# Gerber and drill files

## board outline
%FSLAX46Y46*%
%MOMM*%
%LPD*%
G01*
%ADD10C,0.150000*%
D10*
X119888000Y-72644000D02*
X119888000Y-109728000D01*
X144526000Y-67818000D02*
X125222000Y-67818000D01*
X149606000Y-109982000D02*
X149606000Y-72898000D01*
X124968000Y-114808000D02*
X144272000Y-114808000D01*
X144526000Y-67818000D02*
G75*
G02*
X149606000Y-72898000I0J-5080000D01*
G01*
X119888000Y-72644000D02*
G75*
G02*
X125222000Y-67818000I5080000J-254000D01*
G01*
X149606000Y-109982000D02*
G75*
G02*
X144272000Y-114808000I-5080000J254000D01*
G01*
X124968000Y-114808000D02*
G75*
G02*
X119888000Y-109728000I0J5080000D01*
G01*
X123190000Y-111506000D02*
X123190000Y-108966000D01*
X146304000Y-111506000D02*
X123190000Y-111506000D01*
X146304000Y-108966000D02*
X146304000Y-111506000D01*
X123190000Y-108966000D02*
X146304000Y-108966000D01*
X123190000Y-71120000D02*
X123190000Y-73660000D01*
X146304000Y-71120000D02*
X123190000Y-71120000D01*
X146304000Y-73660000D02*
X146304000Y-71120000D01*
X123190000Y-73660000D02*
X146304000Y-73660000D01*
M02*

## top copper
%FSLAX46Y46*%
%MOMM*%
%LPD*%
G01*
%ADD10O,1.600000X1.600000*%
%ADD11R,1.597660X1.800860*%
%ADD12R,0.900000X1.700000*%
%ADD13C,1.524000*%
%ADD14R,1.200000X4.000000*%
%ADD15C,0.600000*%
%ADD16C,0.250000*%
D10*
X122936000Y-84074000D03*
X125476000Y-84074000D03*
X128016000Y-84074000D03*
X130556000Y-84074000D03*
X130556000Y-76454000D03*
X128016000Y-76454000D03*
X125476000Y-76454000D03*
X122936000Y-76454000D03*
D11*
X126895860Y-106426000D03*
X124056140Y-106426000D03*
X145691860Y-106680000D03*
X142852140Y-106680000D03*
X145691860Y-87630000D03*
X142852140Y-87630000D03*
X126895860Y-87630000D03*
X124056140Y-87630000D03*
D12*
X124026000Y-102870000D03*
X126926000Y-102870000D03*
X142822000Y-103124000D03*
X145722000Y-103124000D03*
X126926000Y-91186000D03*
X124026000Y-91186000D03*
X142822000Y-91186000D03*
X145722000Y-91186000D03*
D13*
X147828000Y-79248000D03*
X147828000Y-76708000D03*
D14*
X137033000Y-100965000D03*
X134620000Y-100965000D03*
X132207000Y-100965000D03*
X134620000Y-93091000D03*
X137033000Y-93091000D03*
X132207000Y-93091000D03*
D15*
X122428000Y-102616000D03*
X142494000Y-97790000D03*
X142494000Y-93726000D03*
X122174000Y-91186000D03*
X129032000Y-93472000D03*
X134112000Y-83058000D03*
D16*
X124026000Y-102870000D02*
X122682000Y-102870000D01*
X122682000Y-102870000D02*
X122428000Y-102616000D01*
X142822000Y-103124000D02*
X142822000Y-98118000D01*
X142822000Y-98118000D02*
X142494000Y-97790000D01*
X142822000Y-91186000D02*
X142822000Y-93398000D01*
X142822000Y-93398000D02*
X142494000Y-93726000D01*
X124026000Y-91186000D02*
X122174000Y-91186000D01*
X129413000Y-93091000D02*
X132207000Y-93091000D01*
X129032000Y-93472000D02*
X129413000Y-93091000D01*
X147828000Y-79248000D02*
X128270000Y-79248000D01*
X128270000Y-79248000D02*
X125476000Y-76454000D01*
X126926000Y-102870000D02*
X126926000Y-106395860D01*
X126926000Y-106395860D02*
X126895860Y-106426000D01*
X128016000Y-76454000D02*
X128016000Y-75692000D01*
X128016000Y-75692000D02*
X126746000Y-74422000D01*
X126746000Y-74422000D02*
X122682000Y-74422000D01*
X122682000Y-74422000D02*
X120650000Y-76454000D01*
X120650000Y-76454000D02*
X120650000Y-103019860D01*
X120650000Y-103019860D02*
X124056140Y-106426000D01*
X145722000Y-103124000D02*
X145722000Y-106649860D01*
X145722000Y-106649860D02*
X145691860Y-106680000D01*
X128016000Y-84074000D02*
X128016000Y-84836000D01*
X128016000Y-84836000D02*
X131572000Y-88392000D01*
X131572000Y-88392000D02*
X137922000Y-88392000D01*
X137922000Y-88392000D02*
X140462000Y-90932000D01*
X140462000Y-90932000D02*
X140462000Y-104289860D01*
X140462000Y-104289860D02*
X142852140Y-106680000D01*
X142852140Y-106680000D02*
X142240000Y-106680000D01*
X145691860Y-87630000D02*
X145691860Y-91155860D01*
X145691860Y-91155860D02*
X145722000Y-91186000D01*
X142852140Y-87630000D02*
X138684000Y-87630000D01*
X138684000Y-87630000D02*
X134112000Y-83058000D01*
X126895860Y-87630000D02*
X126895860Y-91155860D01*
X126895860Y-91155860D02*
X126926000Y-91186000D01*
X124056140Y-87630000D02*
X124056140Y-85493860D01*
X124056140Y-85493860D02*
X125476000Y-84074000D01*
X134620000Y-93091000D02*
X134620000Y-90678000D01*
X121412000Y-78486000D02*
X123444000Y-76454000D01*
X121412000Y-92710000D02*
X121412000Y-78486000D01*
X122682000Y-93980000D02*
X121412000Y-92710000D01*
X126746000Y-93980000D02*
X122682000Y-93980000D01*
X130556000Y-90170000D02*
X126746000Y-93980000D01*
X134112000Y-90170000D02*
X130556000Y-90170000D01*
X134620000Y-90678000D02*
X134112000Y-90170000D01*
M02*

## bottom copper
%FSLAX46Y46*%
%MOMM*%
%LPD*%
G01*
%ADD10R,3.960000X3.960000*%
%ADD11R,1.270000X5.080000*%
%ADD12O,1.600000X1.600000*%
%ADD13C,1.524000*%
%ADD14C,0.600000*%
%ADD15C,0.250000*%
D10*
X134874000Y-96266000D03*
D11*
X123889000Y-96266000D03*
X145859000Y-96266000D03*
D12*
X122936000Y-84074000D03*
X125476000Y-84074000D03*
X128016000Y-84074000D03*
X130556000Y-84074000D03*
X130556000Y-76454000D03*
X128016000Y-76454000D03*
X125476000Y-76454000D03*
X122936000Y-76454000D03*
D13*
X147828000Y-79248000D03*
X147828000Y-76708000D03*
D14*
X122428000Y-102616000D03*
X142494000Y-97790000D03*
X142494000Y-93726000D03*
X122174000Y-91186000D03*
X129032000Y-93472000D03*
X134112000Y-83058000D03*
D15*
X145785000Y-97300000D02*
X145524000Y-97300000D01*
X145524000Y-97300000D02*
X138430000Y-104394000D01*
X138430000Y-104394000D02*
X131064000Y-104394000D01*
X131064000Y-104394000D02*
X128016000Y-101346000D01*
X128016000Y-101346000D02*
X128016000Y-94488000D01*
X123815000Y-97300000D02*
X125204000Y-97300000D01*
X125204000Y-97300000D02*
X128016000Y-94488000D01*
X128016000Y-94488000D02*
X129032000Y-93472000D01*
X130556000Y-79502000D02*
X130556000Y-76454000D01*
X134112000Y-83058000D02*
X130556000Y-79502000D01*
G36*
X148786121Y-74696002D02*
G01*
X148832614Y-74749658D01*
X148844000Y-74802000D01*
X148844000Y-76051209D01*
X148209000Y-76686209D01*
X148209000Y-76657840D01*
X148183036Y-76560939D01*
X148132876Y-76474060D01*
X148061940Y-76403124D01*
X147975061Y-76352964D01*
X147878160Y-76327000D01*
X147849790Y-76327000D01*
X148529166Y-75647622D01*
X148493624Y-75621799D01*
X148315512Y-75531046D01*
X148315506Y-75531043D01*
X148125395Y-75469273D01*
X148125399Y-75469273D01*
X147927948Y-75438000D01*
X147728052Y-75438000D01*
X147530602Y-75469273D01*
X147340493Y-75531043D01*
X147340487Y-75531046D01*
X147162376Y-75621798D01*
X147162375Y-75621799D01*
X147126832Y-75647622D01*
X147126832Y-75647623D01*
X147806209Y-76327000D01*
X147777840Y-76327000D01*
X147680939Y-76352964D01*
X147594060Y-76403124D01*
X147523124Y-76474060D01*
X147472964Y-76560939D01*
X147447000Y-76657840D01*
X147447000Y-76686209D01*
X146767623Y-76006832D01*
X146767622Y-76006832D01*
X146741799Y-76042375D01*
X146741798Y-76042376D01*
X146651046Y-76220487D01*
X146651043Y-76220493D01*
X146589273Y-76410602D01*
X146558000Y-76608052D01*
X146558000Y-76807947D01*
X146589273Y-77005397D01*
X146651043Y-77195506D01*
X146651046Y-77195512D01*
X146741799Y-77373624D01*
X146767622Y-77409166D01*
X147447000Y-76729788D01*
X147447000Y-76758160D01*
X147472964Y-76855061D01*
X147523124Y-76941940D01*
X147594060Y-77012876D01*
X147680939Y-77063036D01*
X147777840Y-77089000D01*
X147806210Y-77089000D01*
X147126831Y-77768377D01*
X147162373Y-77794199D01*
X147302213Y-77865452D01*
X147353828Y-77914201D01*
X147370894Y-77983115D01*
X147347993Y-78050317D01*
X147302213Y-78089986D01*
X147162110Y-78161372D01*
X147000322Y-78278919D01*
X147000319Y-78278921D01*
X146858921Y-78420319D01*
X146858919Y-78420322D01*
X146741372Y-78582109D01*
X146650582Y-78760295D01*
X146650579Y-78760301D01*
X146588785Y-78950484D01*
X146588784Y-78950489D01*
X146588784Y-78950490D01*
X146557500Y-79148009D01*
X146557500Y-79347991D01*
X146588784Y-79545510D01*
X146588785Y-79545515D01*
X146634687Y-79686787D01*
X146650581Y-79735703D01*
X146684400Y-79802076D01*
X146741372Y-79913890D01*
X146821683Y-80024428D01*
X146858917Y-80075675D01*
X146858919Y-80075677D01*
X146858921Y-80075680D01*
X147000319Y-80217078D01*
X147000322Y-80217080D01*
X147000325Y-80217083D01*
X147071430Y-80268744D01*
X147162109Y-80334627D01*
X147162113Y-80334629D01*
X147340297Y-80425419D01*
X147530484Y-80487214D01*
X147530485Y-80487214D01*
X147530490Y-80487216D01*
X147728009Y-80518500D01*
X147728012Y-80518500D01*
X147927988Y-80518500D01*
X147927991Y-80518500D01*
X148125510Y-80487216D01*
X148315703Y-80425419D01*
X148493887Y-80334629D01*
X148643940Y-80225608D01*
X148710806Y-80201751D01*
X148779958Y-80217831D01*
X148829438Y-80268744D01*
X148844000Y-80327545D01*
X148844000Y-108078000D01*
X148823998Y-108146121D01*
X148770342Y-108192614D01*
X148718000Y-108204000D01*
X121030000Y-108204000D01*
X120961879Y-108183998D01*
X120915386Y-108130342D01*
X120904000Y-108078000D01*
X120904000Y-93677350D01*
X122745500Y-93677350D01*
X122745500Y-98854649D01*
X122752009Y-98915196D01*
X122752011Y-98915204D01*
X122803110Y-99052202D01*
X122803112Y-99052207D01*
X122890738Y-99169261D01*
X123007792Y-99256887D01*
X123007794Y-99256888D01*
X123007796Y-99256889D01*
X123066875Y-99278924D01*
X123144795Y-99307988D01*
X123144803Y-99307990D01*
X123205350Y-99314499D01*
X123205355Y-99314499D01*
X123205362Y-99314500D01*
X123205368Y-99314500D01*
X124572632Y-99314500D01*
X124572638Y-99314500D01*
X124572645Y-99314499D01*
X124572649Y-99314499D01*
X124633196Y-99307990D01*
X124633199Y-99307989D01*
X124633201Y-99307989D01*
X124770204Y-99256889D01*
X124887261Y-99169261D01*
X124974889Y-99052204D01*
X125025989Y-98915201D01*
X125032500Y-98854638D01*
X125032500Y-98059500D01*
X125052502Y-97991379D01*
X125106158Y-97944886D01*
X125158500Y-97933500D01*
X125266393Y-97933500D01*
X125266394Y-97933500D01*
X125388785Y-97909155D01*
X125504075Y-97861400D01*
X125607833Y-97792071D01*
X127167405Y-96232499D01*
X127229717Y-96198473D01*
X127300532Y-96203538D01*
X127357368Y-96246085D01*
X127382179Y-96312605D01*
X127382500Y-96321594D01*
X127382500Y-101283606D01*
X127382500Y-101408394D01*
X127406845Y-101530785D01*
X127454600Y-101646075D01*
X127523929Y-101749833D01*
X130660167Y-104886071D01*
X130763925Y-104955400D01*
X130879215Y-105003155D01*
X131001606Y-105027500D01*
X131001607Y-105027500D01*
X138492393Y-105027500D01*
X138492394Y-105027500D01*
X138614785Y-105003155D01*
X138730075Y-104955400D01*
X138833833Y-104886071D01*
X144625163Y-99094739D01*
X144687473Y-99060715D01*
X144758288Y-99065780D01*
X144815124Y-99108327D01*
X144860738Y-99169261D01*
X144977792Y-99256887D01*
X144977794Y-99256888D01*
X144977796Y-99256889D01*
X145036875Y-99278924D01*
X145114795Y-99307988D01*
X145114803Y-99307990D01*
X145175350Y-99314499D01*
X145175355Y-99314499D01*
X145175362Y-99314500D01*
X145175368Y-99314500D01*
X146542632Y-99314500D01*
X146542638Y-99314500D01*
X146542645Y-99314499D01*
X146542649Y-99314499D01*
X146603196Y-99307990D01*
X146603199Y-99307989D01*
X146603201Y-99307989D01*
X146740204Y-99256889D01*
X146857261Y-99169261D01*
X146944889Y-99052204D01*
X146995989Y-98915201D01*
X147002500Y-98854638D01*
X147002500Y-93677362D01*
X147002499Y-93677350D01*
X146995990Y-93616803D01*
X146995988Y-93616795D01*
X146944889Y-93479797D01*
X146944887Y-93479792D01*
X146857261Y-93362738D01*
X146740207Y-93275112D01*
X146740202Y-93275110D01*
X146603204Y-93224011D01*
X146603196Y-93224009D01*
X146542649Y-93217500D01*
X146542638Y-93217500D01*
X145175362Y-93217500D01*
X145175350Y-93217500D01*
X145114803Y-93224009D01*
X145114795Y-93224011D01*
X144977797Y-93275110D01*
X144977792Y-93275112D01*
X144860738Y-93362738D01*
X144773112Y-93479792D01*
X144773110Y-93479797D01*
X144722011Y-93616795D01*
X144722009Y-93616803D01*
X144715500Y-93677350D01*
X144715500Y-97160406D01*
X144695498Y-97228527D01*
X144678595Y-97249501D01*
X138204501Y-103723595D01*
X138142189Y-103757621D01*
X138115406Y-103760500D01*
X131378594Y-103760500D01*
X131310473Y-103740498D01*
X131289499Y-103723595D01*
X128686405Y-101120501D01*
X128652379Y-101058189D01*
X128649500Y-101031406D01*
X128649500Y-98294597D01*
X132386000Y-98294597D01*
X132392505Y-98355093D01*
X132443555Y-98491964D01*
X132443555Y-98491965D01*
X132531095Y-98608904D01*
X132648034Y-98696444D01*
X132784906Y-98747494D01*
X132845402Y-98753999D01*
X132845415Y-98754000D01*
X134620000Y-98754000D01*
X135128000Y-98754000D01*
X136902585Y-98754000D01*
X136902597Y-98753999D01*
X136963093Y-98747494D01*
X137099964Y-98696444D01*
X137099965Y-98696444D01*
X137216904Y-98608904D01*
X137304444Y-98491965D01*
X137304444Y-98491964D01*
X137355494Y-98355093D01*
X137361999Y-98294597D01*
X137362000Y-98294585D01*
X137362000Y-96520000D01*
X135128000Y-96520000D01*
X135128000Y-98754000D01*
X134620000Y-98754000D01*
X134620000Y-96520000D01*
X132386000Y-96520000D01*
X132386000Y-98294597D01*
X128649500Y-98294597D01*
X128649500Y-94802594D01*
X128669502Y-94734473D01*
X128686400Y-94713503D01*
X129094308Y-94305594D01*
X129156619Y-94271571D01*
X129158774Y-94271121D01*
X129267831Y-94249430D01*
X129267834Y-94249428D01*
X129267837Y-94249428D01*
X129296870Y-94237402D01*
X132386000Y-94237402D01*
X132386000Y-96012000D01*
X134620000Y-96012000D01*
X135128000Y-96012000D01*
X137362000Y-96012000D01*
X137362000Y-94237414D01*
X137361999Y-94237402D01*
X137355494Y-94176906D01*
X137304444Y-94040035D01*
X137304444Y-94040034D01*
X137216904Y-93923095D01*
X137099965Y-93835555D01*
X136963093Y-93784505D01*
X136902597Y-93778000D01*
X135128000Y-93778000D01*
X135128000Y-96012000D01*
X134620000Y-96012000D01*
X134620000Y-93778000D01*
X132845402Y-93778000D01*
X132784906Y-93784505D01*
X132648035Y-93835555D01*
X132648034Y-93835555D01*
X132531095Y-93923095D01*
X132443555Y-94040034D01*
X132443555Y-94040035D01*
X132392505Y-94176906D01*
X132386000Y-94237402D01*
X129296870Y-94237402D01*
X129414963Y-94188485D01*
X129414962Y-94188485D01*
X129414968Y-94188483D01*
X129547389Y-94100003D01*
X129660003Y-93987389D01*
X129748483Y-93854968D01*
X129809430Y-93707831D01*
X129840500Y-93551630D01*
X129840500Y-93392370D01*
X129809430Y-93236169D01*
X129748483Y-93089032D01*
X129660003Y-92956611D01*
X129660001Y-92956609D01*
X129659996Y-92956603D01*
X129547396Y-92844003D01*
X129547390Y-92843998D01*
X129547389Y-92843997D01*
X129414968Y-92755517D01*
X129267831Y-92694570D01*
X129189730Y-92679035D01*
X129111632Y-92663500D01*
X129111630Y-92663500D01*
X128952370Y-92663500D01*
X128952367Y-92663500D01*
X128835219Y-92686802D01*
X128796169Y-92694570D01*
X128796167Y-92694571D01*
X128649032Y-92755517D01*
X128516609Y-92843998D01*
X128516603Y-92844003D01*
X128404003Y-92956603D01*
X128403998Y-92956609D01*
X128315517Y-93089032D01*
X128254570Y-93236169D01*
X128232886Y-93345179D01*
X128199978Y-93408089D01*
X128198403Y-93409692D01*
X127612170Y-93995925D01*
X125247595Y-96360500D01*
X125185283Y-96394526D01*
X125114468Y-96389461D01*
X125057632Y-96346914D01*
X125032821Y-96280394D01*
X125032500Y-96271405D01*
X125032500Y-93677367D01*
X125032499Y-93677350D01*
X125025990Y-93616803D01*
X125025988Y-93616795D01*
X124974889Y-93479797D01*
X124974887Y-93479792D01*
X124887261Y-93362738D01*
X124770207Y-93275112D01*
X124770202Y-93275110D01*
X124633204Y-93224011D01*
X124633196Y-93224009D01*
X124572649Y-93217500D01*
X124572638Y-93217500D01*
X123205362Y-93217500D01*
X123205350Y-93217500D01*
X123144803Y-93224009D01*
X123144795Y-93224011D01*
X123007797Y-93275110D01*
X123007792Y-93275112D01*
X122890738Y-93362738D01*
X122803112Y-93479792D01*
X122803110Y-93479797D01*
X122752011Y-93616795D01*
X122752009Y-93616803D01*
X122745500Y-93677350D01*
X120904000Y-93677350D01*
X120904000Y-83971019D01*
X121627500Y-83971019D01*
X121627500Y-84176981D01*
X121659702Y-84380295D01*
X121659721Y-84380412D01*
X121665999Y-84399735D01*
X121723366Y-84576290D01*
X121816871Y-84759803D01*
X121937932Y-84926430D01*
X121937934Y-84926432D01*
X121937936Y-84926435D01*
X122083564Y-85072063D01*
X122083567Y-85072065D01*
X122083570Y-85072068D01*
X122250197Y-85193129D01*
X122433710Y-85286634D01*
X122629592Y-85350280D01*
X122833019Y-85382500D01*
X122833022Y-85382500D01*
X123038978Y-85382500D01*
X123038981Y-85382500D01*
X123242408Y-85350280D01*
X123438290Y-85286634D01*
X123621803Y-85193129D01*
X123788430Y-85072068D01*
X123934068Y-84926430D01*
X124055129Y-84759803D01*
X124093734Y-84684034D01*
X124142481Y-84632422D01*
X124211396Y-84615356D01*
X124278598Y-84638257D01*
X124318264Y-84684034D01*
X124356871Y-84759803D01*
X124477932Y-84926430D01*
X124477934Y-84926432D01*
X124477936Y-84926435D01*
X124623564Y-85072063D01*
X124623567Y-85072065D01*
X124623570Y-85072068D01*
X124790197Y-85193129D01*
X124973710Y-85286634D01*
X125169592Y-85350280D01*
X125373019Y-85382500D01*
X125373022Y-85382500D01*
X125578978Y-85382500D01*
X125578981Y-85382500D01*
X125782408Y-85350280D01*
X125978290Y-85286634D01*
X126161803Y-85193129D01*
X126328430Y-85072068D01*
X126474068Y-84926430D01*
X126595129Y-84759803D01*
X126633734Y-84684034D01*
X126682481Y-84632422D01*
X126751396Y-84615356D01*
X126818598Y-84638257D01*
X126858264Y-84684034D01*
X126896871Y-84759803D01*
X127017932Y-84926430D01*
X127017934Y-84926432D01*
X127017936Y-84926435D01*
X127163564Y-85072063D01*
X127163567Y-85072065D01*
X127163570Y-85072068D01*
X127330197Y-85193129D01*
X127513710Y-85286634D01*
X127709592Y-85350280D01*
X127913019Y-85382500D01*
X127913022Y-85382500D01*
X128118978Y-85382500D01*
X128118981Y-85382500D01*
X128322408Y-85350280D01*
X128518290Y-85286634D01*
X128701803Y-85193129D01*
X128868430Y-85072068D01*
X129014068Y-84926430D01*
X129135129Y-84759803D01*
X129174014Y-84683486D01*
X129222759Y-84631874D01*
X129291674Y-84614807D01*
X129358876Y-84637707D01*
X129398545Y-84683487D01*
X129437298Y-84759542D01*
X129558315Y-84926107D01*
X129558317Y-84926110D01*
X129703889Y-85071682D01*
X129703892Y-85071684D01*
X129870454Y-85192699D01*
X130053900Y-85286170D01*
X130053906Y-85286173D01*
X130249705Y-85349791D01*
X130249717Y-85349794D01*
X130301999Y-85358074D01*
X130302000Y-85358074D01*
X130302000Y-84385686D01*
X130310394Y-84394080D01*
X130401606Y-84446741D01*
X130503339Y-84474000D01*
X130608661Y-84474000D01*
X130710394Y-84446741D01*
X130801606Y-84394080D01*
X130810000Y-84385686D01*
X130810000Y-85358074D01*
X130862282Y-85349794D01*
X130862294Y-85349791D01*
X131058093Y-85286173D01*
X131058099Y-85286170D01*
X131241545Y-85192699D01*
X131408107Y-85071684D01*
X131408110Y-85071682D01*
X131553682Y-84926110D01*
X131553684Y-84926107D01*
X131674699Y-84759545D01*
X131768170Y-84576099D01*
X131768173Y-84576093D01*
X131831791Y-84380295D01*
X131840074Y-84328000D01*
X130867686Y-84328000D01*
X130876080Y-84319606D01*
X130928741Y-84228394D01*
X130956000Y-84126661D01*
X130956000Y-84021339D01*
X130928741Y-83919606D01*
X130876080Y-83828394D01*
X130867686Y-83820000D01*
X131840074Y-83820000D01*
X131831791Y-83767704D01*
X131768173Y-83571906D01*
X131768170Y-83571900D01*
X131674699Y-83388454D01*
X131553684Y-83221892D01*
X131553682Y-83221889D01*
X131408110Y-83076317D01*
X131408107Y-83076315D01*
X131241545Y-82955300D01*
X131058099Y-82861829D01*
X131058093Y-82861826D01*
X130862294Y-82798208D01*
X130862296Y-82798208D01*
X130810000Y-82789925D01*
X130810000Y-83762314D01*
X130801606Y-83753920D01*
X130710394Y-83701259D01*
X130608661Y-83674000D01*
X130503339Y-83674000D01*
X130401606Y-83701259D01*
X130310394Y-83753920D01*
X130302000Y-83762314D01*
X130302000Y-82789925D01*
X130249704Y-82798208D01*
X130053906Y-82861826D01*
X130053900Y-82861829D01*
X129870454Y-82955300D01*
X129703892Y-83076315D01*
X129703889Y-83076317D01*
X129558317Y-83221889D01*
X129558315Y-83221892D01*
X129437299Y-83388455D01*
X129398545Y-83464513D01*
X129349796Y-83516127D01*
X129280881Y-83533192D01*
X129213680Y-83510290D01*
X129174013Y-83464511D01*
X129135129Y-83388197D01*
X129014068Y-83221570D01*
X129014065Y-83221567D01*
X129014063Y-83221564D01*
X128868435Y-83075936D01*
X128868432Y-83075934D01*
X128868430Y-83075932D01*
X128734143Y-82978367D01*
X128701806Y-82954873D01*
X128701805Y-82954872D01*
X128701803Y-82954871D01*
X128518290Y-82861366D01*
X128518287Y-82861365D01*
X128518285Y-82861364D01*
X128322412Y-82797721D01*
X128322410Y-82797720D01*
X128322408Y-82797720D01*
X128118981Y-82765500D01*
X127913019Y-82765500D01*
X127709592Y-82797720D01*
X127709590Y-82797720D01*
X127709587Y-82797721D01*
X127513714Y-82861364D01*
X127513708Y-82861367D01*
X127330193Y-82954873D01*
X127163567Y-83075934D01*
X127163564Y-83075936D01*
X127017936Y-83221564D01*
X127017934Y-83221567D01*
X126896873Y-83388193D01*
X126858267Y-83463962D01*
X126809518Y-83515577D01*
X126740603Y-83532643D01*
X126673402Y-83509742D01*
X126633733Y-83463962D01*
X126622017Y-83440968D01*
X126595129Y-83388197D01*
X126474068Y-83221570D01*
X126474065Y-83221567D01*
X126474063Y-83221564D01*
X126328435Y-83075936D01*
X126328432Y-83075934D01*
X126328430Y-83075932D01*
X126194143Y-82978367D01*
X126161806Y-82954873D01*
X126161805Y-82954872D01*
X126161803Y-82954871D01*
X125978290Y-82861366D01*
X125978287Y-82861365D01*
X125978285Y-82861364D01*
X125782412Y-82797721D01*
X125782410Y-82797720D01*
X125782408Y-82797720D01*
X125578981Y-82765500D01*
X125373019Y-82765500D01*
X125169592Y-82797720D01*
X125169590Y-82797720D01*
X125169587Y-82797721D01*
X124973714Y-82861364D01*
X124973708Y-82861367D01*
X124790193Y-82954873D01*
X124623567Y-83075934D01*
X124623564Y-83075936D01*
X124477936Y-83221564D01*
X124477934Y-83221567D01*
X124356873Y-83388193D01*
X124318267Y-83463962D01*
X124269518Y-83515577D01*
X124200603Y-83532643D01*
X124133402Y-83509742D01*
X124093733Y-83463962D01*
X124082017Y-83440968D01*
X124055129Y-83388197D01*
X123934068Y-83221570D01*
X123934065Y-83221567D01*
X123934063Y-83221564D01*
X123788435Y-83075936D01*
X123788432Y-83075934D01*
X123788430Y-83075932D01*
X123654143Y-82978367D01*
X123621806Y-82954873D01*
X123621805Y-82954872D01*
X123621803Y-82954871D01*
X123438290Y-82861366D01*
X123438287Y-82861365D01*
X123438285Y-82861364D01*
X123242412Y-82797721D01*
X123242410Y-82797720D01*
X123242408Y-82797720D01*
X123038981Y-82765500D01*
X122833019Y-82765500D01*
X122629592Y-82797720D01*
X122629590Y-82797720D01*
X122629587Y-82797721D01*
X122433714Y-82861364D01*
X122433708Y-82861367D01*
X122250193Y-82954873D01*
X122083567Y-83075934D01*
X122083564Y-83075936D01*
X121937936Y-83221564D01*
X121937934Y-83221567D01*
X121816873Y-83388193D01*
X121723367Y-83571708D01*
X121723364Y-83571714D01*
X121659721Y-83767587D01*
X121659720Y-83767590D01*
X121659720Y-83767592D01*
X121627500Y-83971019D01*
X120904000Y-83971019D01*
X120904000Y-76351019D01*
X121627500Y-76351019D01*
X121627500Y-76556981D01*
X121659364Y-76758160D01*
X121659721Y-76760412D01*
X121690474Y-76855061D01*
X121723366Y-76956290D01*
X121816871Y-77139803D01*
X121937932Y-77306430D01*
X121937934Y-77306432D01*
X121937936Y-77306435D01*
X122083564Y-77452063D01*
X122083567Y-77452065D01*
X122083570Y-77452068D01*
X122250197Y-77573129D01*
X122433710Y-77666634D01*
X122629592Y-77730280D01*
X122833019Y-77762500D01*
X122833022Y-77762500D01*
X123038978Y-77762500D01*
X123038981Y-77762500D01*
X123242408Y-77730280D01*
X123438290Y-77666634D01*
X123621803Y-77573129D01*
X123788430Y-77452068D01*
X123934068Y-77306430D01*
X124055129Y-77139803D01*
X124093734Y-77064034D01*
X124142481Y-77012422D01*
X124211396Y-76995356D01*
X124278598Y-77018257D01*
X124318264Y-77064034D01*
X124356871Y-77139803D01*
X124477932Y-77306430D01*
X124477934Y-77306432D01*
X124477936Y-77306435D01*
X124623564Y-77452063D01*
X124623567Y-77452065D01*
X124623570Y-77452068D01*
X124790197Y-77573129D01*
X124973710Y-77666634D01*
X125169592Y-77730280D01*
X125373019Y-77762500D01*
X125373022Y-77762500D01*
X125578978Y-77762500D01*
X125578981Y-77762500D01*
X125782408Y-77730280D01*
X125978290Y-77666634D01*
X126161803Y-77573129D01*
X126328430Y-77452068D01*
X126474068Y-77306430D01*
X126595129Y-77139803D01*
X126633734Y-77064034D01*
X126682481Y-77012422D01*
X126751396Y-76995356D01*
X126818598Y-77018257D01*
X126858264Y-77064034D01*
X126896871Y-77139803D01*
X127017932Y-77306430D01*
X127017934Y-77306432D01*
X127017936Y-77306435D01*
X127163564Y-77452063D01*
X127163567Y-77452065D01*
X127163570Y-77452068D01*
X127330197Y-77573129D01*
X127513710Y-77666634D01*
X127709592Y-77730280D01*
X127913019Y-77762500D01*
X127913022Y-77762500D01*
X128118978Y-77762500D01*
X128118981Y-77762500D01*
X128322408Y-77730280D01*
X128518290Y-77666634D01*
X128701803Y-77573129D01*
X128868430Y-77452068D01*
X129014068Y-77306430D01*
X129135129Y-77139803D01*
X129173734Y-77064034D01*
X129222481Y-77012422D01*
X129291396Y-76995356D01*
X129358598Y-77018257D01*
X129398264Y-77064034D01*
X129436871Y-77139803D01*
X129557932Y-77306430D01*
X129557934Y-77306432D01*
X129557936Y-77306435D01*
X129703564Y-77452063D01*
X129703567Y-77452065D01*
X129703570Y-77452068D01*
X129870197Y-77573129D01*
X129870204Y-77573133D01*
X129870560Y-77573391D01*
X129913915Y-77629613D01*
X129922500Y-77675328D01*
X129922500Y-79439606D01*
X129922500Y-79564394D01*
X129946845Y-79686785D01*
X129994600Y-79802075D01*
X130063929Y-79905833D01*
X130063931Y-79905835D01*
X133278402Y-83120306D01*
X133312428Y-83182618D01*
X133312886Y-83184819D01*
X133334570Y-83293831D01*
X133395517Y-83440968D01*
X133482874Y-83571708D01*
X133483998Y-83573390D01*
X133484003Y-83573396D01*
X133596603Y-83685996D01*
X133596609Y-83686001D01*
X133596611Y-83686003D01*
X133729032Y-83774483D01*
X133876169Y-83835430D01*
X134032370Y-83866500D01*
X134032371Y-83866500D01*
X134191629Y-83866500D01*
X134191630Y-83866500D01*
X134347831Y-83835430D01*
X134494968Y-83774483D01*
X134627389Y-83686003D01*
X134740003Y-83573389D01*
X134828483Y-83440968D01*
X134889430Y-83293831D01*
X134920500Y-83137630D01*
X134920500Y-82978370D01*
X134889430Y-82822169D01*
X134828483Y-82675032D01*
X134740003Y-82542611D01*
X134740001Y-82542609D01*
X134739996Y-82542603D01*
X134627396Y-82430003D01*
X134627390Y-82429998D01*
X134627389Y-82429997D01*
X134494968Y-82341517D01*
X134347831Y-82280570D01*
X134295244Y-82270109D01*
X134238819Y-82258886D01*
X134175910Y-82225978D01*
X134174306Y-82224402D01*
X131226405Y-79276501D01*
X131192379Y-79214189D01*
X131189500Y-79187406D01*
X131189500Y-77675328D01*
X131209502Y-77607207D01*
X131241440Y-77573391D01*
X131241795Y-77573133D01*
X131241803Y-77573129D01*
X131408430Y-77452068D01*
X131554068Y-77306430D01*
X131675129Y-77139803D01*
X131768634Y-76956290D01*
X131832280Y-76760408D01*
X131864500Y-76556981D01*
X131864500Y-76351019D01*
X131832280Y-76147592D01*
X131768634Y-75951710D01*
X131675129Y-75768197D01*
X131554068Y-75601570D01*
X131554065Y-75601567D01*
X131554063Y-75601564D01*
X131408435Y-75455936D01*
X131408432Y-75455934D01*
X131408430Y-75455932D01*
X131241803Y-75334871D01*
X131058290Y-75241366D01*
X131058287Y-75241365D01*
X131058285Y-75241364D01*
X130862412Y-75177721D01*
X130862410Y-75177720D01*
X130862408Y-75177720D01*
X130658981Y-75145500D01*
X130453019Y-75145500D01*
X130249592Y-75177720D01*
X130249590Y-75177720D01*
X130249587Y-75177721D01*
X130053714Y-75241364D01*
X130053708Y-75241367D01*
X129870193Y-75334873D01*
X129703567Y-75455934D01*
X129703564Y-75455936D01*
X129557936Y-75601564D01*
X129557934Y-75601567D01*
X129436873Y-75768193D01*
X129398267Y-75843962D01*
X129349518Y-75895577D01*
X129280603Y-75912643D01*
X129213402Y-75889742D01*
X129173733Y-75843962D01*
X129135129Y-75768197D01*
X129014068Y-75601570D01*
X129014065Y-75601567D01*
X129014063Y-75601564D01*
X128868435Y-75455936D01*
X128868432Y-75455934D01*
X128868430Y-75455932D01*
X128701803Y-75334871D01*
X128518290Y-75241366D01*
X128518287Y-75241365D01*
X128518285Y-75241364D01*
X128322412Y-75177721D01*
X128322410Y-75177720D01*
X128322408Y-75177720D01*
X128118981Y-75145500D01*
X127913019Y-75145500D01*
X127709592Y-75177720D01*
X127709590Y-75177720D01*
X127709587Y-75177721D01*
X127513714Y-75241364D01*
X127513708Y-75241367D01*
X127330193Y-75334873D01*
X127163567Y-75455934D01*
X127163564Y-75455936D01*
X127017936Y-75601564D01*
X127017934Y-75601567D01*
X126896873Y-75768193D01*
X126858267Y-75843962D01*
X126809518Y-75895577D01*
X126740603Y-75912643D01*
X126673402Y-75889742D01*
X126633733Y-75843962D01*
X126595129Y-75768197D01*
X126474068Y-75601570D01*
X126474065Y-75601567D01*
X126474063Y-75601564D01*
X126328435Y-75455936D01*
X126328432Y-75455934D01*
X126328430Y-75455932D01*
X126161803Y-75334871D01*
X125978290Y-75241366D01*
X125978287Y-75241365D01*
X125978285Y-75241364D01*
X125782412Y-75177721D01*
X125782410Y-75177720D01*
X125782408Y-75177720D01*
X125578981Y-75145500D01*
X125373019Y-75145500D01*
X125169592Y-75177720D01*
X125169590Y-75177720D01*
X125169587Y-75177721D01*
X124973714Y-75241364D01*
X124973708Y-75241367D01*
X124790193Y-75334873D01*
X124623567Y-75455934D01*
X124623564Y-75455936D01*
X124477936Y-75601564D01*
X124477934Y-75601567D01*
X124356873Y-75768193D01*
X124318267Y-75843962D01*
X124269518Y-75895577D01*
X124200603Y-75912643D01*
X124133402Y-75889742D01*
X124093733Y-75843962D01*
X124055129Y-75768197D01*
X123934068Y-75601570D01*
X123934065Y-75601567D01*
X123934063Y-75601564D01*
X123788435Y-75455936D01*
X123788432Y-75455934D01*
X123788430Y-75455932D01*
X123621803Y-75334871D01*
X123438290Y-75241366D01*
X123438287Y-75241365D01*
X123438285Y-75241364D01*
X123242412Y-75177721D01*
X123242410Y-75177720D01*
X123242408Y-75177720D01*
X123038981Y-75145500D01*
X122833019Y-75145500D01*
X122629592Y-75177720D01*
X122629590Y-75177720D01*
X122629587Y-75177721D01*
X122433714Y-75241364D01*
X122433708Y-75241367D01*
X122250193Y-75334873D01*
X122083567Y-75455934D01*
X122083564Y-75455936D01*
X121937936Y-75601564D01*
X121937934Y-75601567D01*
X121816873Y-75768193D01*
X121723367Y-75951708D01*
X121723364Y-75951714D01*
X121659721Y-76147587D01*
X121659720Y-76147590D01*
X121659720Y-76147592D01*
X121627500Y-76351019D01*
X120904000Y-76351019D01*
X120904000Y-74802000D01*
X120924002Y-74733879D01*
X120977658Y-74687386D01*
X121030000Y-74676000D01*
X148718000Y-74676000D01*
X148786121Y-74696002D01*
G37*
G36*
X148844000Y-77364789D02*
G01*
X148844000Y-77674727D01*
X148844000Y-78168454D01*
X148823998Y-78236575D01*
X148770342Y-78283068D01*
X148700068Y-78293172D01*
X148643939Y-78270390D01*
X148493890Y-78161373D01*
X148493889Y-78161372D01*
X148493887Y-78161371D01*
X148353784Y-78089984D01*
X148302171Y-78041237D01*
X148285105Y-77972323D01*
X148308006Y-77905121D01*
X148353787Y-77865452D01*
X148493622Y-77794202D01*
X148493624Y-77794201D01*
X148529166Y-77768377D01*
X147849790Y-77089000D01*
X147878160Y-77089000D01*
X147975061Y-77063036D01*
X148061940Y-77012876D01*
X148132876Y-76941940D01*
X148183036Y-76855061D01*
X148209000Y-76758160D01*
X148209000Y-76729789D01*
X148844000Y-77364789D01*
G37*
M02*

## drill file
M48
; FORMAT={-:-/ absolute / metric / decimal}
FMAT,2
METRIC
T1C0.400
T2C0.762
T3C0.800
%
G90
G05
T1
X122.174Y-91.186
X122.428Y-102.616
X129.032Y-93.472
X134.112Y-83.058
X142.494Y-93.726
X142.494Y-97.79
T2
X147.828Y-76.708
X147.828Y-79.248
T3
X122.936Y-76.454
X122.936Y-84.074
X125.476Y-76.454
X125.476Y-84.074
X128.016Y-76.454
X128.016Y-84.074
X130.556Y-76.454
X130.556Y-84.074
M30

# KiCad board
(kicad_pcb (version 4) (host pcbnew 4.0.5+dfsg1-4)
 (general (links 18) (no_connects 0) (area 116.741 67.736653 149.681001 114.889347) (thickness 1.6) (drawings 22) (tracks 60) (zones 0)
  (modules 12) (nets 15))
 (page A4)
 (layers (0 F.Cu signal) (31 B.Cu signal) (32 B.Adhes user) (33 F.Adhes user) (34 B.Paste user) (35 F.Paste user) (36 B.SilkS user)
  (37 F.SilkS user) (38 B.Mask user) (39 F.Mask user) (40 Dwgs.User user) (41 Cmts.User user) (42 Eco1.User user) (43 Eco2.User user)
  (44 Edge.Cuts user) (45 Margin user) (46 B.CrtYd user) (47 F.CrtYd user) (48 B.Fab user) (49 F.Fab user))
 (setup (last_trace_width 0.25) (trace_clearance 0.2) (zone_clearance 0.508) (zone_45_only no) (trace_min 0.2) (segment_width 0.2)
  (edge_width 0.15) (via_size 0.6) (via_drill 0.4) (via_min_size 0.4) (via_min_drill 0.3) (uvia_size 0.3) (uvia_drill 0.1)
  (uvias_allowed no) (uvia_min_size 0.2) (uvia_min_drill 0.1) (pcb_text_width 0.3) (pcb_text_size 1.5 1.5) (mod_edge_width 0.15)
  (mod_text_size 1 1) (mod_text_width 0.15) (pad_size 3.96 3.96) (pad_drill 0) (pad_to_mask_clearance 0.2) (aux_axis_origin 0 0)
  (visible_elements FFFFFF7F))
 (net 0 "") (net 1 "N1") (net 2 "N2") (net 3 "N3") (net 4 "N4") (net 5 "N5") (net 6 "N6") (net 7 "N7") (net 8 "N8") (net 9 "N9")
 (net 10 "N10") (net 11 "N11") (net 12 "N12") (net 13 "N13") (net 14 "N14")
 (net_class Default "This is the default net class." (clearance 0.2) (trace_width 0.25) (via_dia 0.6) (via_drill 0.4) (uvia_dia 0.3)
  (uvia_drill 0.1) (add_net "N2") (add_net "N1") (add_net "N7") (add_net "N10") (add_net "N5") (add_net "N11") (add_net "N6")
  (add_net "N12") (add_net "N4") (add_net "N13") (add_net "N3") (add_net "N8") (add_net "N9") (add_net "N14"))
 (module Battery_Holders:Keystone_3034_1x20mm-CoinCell (layer B.Cu) (at 134.874 96.266 180)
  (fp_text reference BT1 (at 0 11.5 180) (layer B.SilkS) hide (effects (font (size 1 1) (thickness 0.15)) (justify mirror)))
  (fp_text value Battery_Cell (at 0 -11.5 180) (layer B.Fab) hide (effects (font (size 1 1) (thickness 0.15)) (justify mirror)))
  (pad 2 smd rect (at 0 0 180) (size 3.96 3.96) (layers B.Cu B.Paste B.Mask) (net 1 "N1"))
  (pad 1 smd rect (at 10.985 0 180) (size 1.27 5.08) (layers B.Cu B.Paste B.Mask) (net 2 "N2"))
  (pad 1 smd rect (at -10.985 0 180) (size 1.27 5.08) (layers B.Cu B.Paste B.Mask) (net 2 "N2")))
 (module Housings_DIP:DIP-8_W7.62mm (layer F.Cu) (at 122.936 84.074 90)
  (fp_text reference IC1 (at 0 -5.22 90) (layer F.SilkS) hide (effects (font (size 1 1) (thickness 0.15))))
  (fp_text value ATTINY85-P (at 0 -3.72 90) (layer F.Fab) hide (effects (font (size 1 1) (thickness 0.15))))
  (pad 1 thru_hole oval (at 0 0 90) (size 1.6 1.6) (drill 0.8) (layers *.Cu *.Mask) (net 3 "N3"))
  (pad 2 thru_hole oval (at 0 2.54 90) (size 1.6 1.6) (drill 0.8) (layers *.Cu *.Mask) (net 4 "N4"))
  (pad 3 thru_hole oval (at 0 5.08 90) (size 1.6 1.6) (drill 0.8) (layers *.Cu *.Mask) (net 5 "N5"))
  (pad 4 thru_hole oval (at 0 7.62 90) (size 1.6 1.6) (drill 0.8) (layers *.Cu *.Mask) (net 1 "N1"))
  (pad 5 thru_hole oval (at 7.62 7.62 90) (size 1.6 1.6) (drill 0.8) (layers *.Cu *.Mask) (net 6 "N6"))
  (pad 6 thru_hole oval (at 7.62 5.08 90) (size 1.6 1.6) (drill 0.8) (layers *.Cu *.Mask) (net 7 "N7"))
  (pad 7 thru_hole oval (at 7.62 2.54 90) (size 1.6 1.6) (drill 0.8) (layers *.Cu *.Mask) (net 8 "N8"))
  (pad 8 thru_hole oval (at 7.62 0 90) (size 1.6 1.6) (drill 0.8) (layers *.Cu *.Mask) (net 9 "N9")))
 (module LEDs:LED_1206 (layer F.Cu) (at 125.476 106.426)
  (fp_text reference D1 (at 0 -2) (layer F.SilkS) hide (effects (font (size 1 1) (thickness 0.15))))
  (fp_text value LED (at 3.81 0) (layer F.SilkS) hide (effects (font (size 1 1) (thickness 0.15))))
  (pad 2 smd rect (at 1.41986 0 180) (size 1.59766 1.80086) (layers F.Cu F.Paste F.Mask) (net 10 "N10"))
  (pad 1 smd rect (at -1.41986 0 180) (size 1.59766 1.80086) (layers F.Cu F.Paste F.Mask) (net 7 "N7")))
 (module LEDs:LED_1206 (layer F.Cu) (at 144.272 106.68)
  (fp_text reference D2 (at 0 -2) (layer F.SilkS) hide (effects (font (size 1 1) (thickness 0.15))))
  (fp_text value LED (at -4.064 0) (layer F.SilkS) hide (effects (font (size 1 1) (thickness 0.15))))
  (pad 2 smd rect (at 1.41986 0 180) (size 1.59766 1.80086) (layers F.Cu F.Paste F.Mask) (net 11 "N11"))
  (pad 1 smd rect (at -1.41986 0 180) (size 1.59766 1.80086) (layers F.Cu F.Paste F.Mask) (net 5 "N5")))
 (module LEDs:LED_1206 (layer F.Cu) (at 144.272 87.63)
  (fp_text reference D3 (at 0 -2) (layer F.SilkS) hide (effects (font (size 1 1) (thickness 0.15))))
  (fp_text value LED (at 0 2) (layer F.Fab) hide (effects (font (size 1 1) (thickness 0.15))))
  (pad 2 smd rect (at 1.41986 0 180) (size 1.59766 1.80086) (layers F.Cu F.Paste F.Mask) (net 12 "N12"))
  (pad 1 smd rect (at -1.41986 0 180) (size 1.59766 1.80086) (layers F.Cu F.Paste F.Mask) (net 6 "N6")))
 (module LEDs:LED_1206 (layer F.Cu) (at 125.476 87.63)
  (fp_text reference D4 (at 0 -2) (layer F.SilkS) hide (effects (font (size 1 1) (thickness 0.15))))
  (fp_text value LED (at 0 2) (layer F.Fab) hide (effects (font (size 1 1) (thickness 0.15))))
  (pad 2 smd rect (at 1.41986 0 180) (size 1.59766 1.80086) (layers F.Cu F.Paste F.Mask) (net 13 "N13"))
  (pad 1 smd rect (at -1.41986 0 180) (size 1.59766 1.80086) (layers F.Cu F.Paste F.Mask) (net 4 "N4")))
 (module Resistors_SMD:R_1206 (layer F.Cu) (at 125.476 102.87)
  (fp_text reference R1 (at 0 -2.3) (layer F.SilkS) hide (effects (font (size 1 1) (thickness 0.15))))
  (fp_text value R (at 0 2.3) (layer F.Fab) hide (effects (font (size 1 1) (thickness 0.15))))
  (pad 1 smd rect (at -1.45 0) (size 0.9 1.7) (layers F.Cu F.Paste F.Mask) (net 1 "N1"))
  (pad 2 smd rect (at 1.45 0) (size 0.9 1.7) (layers F.Cu F.Paste F.Mask) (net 10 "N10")))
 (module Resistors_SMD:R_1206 (layer F.Cu) (at 144.272 103.124)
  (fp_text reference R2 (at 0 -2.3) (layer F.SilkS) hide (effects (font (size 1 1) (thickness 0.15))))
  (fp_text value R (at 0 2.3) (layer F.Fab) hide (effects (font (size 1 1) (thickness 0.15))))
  (pad 1 smd rect (at -1.45 0) (size 0.9 1.7) (layers F.Cu F.Paste F.Mask) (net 1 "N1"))
  (pad 2 smd rect (at 1.45 0) (size 0.9 1.7) (layers F.Cu F.Paste F.Mask) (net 11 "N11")))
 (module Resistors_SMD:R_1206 (layer F.Cu) (at 125.476 91.186 180)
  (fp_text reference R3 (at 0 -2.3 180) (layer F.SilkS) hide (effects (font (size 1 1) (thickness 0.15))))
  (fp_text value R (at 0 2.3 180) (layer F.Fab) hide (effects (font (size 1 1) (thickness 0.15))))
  (pad 1 smd rect (at -1.45 0 180) (size 0.9 1.7) (layers F.Cu F.Paste F.Mask) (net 13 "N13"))
  (pad 2 smd rect (at 1.45 0 180) (size 0.9 1.7) (layers F.Cu F.Paste F.Mask) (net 1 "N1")))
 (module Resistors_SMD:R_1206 (layer F.Cu) (at 144.272 91.186)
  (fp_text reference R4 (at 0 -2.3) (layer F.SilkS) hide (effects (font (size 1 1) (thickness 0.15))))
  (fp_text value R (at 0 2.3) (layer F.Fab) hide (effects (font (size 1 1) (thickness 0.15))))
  (pad 1 smd rect (at -1.45 0) (size 0.9 1.7) (layers F.Cu F.Paste F.Mask) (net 1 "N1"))
  (pad 2 smd rect (at 1.45 0) (size 0.9 1.7) (layers F.Cu F.Paste F.Mask) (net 12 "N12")))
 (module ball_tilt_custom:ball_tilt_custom (layer F.Cu) (at 147.828 77.978 180)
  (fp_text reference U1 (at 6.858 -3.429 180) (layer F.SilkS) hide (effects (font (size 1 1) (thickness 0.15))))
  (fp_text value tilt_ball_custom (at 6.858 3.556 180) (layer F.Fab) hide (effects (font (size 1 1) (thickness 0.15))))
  (pad 1 thru_hole circle (at 0 -1.27 180) (size 1.524 1.524) (drill 0.762) (layers *.Cu *.Mask) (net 8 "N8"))
  (pad 2 thru_hole circle (at 0 1.27 180) (size 1.524 1.524) (drill 0.762) (layers *.Cu *.Mask) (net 1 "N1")))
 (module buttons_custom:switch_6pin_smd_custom (layer F.Cu) (at 134.62 97.028)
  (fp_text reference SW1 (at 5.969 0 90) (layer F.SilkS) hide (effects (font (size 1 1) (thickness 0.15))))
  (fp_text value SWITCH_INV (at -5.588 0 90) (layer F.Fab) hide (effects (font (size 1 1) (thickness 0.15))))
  (pad 6 smd rect (at 2.413 3.937) (size 1.2 4) (layers F.Cu F.Paste F.Mask))
  (pad 5 smd rect (at 0 3.937) (size 1.2 4) (layers F.Cu F.Paste F.Mask))
  (pad 4 smd rect (at -2.413 3.937) (size 1.2 4) (layers F.Cu F.Paste F.Mask))
  (pad 2 smd rect (at 0 -3.937) (size 1.2 4) (layers F.Cu F.Paste F.Mask) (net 9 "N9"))
  (pad 3 smd rect (at 2.413 -3.937) (size 1.2 4) (layers F.Cu F.Paste F.Mask) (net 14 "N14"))
  (pad 1 smd rect (at -2.413 -3.937) (size 1.2 4) (layers F.Cu F.Paste F.Mask) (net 2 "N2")))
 (gr_line (start 119.888 72.644) (end 119.888 109.728) (angle 90) (layer Edge.Cuts) (width 0.15))
 (gr_line (start 144.526 67.818) (end 125.222 67.818) (angle 90) (layer Edge.Cuts) (width 0.15))
 (gr_line (start 149.606 109.982) (end 149.606 72.898) (angle 90) (layer Edge.Cuts) (width 0.15))
 (gr_line (start 124.968 114.808) (end 144.272 114.808) (angle 90) (layer Edge.Cuts) (width 0.15))
 (gr_arc (start 144.526 72.898) (end 144.526 67.818) (angle 90) (layer Edge.Cuts) (width 0.15))
 (gr_arc (start 124.968 72.898) (end 119.888 72.644) (angle 90) (layer Edge.Cuts) (width 0.15))
 (gr_arc (start 144.526 109.728) (end 149.606 109.982) (angle 90) (layer Edge.Cuts) (width 0.15))
 (gr_arc (start 124.968 109.728) (end 124.968 114.808) (angle 90) (layer Edge.Cuts) (width 0.15))
 (gr_line (start 123.19 111.506) (end 123.19 108.966) (angle 90) (layer Edge.Cuts) (width 0.15))
 (gr_line (start 146.304 111.506) (end 123.19 111.506) (angle 90) (layer Edge.Cuts) (width 0.15))
 (gr_line (start 146.304 108.966) (end 146.304 111.506) (angle 90) (layer Edge.Cuts) (width 0.15))
 (gr_line (start 123.19 108.966) (end 146.304 108.966) (angle 90) (layer Edge.Cuts) (width 0.15))
 (gr_line (start 123.19 71.12) (end 123.19 73.66) (angle 90) (layer Edge.Cuts) (width 0.15))
 (gr_line (start 146.304 71.12) (end 123.19 71.12) (angle 90) (layer Edge.Cuts) (width 0.15))
 (gr_line (start 146.304 73.66) (end 146.304 71.12) (angle 90) (layer Edge.Cuts) (width 0.15))
 (gr_line (start 123.19 73.66) (end 146.304 73.66) (angle 90) (layer Edge.Cuts) (width 0.15))
 (segment (start 124.026 102.87) (end 122.682 102.87) (width 0.25) (layer F.Cu) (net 1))
 (via (at 122.428 102.616) (size 0.6) (drill 0.4) (layers F.Cu B.Cu) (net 1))
 (segment (start 122.682 102.87) (end 122.428 102.616) (width 0.25) (layer F.Cu) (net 1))
 (segment (start 142.822 103.124) (end 142.822 98.118) (width 0.25) (layer F.Cu) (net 1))
 (via (at 142.494 97.79) (size 0.6) (drill 0.4) (layers F.Cu B.Cu) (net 1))
 (segment (start 142.822 98.118) (end 142.494 97.79) (width 0.25) (layer F.Cu) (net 1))
 (segment (start 142.822 91.186) (end 142.822 93.398) (width 0.25) (layer F.Cu) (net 1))
 (via (at 142.494 93.726) (size 0.6) (drill 0.4) (layers F.Cu B.Cu) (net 1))
 (segment (start 142.822 93.398) (end 142.494 93.726) (width 0.25) (layer F.Cu) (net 1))
 (segment (start 124.026 91.186) (end 122.174 91.186) (width 0.25) (layer F.Cu) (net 1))
 (via (at 122.174 91.186) (size 0.6) (drill 0.4) (layers F.Cu B.Cu) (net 1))
 (segment (start 145.785 97.3) (end 145.524 97.3) (width 0.25) (layer B.Cu) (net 2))
 (segment (start 145.524 97.3) (end 138.43 104.394) (width 0.25) (layer B.Cu) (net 2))
 (segment (start 138.43 104.394) (end 131.064 104.394) (width 0.25) (layer B.Cu) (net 2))
 (segment (start 131.064 104.394) (end 128.016 101.346) (width 0.25) (layer B.Cu) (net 2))
 (segment (start 128.016 101.346) (end 128.016 94.488) (width 0.25) (layer B.Cu) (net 2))
 (segment (start 123.815 97.3) (end 125.204 97.3) (width 0.25) (layer B.Cu) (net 2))
 (segment (start 129.413 93.091) (end 132.207 93.091) (width 0.25) (layer F.Cu) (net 2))
 (segment (start 129.032 93.472) (end 129.413 93.091) (width 0.25) (layer F.Cu) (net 2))
 (via (at 129.032 93.472) (size 0.6) (drill 0.4) (layers F.Cu B.Cu) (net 2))
 (segment (start 125.204 97.3) (end 128.016 94.488) (width 0.25) (layer B.Cu) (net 2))
 (segment (start 128.016 94.488) (end 129.032 93.472) (width 0.25) (layer B.Cu) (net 2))
 (segment (start 147.828 79.248) (end 128.27 79.248) (width 0.25) (layer F.Cu) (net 8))
 (segment (start 128.27 79.248) (end 125.476 76.454) (width 0.25) (layer F.Cu) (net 8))
 (segment (start 126.926 102.87) (end 126.926 106.39586) (width 0.25) (layer F.Cu) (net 10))
 (segment (start 126.926 106.39586) (end 126.89586 106.426) (width 0.25) (layer F.Cu) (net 10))
 (segment (start 128.016 76.454) (end 128.016 75.692) (width 0.25) (layer F.Cu) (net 7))
 (segment (start 128.016 75.692) (end 126.746 74.422) (width 0.25) (layer F.Cu) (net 7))
 (segment (start 126.746 74.422) (end 122.682 74.422) (width 0.25) (layer F.Cu) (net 7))
 (segment (start 122.682 74.422) (end 120.65 76.454) (width 0.25) (layer F.Cu) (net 7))
 (segment (start 120.65 76.454) (end 120.65 103.01986) (width 0.25) (layer F.Cu) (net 7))
 (segment (start 120.65 103.01986) (end 124.05614 106.426) (width 0.25) (layer F.Cu) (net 7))
 (segment (start 145.722 103.124) (end 145.722 106.64986) (width 0.25) (layer F.Cu) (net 11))
 (segment (start 145.722 106.64986) (end 145.69186 106.68) (width 0.25) (layer F.Cu) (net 11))
 (segment (start 128.016 84.074) (end 128.016 84.836) (width 0.25) (layer F.Cu) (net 5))
 (segment (start 128.016 84.836) (end 131.572 88.392) (width 0.25) (layer F.Cu) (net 5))
 (segment (start 131.572 88.392) (end 137.922 88.392) (width 0.25) (layer F.Cu) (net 5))
 (segment (start 137.922 88.392) (end 140.462 90.932) (width 0.25) (layer F.Cu) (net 5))
 (segment (start 140.462 90.932) (end 140.462 104.28986) (width 0.25) (layer F.Cu) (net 5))
 (segment (start 140.462 104.28986) (end 142.85214 106.68) (width 0.25) (layer F.Cu) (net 5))
 (segment (start 142.85214 106.68) (end 142.24 106.68) (width 0.25) (layer F.Cu) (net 5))
 (segment (start 145.69186 87.63) (end 145.69186 91.15586) (width 0.25) (layer F.Cu) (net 12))
 (segment (start 145.69186 91.15586) (end 145.722 91.186) (width 0.25) (layer F.Cu) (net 12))
 (segment (start 142.85214 87.63) (end 138.684 87.63) (width 0.25) (layer F.Cu) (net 6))
 (segment (start 130.556 79.502) (end 130.556 76.454) (width 0.25) (layer B.Cu) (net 6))
 (segment (start 134.112 83.058) (end 130.556 79.502) (width 0.25) (layer B.Cu) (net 6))
 (via (at 134.112 83.058) (size 0.6) (drill 0.4) (layers F.Cu B.Cu) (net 6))
 (segment (start 138.684 87.63) (end 134.112 83.058) (width 0.25) (layer F.Cu) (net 6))
 (segment (start 126.89586 87.63) (end 126.89586 91.15586) (width 0.25) (layer F.Cu) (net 13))
 (segment (start 126.89586 91.15586) (end 126.926 91.186) (width 0.25) (layer F.Cu) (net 13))
 (segment (start 124.05614 87.63) (end 124.05614 85.49386) (width 0.25) (layer F.Cu) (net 4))
 (segment (start 124.05614 85.49386) (end 125.476 84.074) (width 0.25) (layer F.Cu) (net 4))
 (segment (start 134.62 93.091) (end 134.62 90.678) (width 0.25) (layer F.Cu) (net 9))
 (segment (start 121.412 78.486) (end 123.444 76.454) (width 0.25) (layer F.Cu) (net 9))
 (segment (start 121.412 92.71) (end 121.412 78.486) (width 0.25) (layer F.Cu) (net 9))
 (segment (start 122.682 93.98) (end 121.412 92.71) (width 0.25) (layer F.Cu) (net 9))
 (segment (start 126.746 93.98) (end 122.682 93.98) (width 0.25) (layer F.Cu) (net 9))
 (segment (start 130.556 90.17) (end 126.746 93.98) (width 0.25) (layer F.Cu) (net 9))
 (segment (start 134.112 90.17) (end 130.556 90.17) (width 0.25) (layer F.Cu) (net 9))
 (segment (start 134.62 90.678) (end 134.112 90.17) (width 0.25) (layer F.Cu) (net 9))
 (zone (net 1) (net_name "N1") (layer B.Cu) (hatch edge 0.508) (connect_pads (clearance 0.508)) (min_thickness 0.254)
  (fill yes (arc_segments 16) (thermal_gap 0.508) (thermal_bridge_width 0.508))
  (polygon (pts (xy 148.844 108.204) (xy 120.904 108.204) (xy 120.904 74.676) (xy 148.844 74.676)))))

